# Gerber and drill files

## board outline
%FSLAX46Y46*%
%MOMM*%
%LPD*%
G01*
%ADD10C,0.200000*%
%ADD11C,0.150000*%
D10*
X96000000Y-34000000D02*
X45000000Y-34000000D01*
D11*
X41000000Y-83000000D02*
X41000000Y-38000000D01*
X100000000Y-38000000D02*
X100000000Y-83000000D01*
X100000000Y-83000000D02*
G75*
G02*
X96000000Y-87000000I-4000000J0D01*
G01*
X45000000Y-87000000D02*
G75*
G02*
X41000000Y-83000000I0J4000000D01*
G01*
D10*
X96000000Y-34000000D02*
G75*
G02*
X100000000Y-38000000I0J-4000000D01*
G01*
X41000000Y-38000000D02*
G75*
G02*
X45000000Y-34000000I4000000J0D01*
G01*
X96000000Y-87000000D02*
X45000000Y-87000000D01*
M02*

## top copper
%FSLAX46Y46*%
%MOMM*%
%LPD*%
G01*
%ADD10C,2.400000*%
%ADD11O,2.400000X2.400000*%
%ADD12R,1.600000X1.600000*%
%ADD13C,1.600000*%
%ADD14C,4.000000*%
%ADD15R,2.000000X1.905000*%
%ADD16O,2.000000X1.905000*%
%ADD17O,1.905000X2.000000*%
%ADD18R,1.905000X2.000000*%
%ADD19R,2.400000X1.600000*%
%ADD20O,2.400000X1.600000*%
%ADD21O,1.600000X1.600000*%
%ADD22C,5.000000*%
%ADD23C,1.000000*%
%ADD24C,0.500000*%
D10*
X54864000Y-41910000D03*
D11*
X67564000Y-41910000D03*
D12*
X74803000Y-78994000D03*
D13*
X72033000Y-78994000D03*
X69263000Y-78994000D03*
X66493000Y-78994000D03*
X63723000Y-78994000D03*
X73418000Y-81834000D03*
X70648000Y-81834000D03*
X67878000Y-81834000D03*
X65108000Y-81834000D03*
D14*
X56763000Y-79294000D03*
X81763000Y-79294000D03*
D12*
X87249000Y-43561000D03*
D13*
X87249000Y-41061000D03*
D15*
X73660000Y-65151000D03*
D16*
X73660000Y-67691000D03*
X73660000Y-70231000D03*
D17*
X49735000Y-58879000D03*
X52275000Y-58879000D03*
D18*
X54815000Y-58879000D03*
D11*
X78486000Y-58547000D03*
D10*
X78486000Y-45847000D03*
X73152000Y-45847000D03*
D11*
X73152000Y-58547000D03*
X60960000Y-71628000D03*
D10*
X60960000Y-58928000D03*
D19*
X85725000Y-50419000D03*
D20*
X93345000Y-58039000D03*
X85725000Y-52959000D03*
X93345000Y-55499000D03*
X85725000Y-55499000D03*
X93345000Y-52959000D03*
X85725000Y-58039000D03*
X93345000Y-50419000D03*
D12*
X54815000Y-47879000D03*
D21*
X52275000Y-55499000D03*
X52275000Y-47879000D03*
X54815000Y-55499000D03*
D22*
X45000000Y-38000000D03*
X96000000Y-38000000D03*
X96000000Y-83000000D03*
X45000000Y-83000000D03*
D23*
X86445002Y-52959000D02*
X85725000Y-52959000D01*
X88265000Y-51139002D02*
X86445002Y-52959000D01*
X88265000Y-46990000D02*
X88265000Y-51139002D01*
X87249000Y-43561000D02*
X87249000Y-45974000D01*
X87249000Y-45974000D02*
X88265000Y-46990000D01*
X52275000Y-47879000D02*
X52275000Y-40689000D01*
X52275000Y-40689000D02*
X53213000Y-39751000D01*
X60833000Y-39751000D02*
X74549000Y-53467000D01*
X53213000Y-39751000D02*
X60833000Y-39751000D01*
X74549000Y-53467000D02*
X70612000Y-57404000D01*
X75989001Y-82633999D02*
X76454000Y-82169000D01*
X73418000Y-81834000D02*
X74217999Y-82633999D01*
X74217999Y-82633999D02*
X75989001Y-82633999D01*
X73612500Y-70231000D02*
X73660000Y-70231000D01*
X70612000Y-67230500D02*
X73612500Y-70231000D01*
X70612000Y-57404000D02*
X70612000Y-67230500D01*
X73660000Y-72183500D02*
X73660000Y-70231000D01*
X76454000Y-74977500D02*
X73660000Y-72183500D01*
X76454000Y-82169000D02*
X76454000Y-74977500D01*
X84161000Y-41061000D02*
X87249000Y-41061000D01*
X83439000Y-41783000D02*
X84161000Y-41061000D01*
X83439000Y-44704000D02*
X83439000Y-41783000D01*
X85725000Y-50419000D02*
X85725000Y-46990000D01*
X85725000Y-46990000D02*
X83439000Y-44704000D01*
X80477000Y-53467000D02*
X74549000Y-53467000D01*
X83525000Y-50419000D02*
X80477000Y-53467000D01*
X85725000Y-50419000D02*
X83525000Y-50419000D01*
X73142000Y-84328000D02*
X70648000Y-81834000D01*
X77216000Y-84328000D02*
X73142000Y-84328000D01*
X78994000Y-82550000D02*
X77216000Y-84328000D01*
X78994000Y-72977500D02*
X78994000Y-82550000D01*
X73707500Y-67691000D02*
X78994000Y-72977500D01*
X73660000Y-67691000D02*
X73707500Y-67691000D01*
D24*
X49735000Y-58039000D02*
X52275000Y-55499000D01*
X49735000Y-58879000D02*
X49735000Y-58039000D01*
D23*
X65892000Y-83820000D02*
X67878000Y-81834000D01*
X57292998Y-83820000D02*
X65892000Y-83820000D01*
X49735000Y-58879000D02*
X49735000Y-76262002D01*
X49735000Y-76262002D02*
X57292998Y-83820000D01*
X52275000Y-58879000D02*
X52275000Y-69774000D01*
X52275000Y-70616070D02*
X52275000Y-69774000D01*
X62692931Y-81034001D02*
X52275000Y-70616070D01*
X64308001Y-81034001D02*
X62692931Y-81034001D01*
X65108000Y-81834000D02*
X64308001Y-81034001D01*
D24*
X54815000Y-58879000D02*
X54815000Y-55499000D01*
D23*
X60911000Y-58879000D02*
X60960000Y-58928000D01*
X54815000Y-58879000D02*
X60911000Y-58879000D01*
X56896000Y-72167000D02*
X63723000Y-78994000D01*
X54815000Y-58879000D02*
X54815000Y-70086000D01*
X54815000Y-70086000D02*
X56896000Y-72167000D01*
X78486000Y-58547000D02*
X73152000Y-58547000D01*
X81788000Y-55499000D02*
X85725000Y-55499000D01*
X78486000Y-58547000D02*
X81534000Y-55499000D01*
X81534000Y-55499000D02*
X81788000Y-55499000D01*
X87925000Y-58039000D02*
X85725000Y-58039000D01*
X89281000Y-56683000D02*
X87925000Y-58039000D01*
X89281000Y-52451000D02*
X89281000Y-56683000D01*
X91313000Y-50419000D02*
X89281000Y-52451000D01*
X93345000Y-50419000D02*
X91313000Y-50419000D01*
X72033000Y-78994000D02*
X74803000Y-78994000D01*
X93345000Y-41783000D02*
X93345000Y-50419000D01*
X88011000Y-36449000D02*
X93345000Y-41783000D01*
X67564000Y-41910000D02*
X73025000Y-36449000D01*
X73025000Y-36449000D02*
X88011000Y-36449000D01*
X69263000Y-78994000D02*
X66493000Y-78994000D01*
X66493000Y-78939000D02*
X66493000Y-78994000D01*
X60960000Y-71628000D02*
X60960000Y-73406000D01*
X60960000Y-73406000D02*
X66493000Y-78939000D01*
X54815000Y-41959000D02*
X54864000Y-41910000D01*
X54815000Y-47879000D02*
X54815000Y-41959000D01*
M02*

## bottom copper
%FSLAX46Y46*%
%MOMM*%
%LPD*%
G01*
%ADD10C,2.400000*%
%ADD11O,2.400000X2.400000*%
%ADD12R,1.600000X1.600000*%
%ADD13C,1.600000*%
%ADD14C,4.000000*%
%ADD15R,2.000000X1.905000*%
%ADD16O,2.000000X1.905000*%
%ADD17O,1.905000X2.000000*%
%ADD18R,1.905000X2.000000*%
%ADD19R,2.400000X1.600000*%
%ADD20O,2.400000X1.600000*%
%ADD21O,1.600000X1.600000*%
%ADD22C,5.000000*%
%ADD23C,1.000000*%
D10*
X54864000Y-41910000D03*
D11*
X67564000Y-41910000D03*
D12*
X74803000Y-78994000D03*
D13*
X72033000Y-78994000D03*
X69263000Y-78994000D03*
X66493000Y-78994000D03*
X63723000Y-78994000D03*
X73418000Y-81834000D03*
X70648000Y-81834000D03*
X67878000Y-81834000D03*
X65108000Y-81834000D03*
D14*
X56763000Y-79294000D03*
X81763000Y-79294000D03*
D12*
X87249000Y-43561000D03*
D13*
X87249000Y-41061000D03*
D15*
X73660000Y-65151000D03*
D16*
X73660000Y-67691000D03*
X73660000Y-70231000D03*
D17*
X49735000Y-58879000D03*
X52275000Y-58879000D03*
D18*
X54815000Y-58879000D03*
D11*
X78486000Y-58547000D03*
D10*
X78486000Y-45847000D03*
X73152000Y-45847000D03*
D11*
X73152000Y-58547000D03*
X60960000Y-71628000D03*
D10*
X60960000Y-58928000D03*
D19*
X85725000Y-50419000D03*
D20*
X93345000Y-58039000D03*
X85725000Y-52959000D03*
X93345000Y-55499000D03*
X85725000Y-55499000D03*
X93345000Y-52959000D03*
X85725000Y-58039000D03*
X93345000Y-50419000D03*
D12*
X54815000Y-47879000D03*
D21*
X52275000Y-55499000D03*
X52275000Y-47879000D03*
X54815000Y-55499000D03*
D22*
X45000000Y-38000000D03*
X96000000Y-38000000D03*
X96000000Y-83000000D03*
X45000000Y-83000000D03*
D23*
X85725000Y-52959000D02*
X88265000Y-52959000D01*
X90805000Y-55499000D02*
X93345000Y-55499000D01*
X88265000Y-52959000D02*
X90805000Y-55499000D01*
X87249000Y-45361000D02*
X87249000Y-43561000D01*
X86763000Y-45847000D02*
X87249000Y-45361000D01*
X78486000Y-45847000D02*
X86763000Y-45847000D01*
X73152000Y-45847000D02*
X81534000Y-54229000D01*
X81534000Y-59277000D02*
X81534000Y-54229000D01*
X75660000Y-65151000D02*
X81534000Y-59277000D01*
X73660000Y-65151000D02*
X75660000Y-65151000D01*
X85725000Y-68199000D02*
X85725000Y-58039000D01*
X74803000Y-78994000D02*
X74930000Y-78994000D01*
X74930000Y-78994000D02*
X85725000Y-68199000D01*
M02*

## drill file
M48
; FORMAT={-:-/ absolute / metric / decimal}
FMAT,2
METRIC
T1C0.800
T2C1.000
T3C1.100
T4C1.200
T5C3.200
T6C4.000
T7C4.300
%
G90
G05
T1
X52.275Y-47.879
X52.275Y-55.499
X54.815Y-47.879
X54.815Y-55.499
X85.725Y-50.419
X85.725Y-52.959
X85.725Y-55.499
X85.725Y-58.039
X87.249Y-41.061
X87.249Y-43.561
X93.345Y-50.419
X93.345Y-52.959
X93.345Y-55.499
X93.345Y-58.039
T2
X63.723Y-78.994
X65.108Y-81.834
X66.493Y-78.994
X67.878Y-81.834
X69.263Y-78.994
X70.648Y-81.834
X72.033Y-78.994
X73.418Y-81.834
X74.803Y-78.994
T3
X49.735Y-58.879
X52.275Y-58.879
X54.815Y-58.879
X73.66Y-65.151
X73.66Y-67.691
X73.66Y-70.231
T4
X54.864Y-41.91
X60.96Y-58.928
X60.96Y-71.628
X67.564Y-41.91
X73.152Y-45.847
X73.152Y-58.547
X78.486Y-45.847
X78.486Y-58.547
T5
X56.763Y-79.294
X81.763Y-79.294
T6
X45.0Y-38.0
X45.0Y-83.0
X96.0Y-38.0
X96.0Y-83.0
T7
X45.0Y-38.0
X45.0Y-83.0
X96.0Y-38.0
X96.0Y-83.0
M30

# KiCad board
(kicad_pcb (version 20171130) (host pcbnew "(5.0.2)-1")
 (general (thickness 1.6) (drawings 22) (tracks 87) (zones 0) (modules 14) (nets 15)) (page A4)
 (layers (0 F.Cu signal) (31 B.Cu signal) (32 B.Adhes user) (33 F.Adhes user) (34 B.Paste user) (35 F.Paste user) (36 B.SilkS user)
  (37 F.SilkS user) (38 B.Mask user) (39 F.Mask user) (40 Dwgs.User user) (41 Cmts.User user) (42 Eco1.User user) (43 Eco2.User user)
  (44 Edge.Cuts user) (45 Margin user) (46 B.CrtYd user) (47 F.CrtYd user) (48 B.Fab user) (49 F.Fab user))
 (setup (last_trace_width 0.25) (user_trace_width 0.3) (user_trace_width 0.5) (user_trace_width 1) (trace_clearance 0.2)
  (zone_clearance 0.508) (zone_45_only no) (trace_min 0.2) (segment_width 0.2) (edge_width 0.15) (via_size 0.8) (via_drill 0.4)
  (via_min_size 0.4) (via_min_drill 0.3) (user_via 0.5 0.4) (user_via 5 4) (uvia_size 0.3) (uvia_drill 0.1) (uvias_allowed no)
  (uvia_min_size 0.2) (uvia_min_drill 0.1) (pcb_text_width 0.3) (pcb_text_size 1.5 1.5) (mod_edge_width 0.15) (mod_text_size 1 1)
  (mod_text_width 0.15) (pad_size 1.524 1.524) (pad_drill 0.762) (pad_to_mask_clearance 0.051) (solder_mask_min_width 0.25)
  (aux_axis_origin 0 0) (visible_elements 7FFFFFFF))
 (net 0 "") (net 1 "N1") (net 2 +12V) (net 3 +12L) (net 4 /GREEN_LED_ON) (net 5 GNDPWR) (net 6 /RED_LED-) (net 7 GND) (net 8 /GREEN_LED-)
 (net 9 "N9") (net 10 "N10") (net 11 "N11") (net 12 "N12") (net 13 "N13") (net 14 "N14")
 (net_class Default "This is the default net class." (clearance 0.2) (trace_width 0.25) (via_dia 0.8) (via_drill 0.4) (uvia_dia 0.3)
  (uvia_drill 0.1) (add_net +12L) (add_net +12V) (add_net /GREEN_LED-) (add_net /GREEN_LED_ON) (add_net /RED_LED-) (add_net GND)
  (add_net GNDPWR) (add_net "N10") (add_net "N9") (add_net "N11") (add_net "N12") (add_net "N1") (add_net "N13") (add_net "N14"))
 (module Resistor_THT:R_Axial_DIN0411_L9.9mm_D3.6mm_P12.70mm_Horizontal (layer F.Cu) (at 54.864 41.91)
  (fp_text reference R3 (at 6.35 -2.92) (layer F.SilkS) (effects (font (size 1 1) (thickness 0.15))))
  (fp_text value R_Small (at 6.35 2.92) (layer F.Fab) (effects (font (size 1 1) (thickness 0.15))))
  (pad 1 thru_hole circle (at 0 0) (size 2.4 2.4) (drill 1.2) (layers *.Cu *.Mask) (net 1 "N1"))
  (pad 2 thru_hole oval (at 12.7 0) (size 2.4 2.4) (drill 1.2) (layers *.Cu *.Mask) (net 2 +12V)))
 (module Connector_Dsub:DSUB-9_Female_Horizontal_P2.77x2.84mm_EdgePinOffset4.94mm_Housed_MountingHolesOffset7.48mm (layer F.Cu)
  (at 74.803 78.994)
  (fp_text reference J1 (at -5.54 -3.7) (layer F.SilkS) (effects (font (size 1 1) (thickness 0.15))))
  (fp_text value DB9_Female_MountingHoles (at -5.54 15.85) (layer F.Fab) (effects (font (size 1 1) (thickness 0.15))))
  (pad 1 thru_hole rect (at 0 0) (size 1.6 1.6) (drill 1) (layers *.Cu *.Mask) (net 2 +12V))
  (pad 2 thru_hole circle (at -2.77 0) (size 1.6 1.6) (drill 1) (layers *.Cu *.Mask) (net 2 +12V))
  (pad 3 thru_hole circle (at -5.54 0) (size 1.6 1.6) (drill 1) (layers *.Cu *.Mask) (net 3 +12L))
  (pad 4 thru_hole circle (at -8.31 0) (size 1.6 1.6) (drill 1) (layers *.Cu *.Mask) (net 3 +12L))
  (pad 5 thru_hole circle (at -11.08 0) (size 1.6 1.6) (drill 1) (layers *.Cu *.Mask) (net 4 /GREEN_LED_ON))
  (pad 6 thru_hole circle (at -1.385 2.84) (size 1.6 1.6) (drill 1) (layers *.Cu *.Mask) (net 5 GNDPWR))
  (pad 7 thru_hole circle (at -4.155 2.84) (size 1.6 1.6) (drill 1) (layers *.Cu *.Mask) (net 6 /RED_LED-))
  (pad 8 thru_hole circle (at -6.925 2.84) (size 1.6 1.6) (drill 1) (layers *.Cu *.Mask) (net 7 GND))
  (pad 9 thru_hole circle (at -9.695 2.84) (size 1.6 1.6) (drill 1) (layers *.Cu *.Mask) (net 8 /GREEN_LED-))
  (pad 0 thru_hole circle (at -18.04 0.3) (size 4 4) (drill 3.2) (layers *.Cu *.Mask) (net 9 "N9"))
  (pad 0 thru_hole circle (at 6.96 0.3) (size 4 4) (drill 3.2) (layers *.Cu *.Mask) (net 9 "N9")))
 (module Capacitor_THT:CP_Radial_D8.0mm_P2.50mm (layer F.Cu) (at 87.249 43.561 90)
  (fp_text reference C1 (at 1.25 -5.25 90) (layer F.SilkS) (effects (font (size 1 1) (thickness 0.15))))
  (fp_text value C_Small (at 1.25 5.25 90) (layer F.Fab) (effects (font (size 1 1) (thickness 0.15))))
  (pad 1 thru_hole rect (at 0 0 90) (size 1.6 1.6) (drill 0.8) (layers *.Cu *.Mask) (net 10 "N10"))
  (pad 2 thru_hole circle (at 2.5 0 90) (size 1.6 1.6) (drill 0.8) (layers *.Cu *.Mask) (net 5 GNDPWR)))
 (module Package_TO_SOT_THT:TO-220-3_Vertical (layer F.Cu) (at 73.66 65.151 270)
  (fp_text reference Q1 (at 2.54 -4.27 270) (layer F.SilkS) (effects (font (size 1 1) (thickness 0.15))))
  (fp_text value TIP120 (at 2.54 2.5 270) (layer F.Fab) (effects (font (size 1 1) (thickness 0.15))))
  (pad 1 thru_hole rect (at 0 0 270) (size 1.905 2) (drill 1.1) (layers *.Cu *.Mask) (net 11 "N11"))
  (pad 2 thru_hole oval (at 2.54 0 270) (size 1.905 2) (drill 1.1) (layers *.Cu *.Mask) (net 6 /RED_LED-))
  (pad 3 thru_hole oval (at 5.08 0 270) (size 1.905 2) (drill 1.1) (layers *.Cu *.Mask) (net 5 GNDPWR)))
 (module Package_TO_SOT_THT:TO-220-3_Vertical (layer F.Cu) (at 54.815 58.879 180)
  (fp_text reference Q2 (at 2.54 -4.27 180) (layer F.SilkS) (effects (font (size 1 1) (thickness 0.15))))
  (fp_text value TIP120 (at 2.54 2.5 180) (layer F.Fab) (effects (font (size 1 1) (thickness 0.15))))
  (pad 3 thru_hole oval (at 5.08 0 180) (size 1.905 2) (drill 1.1) (layers *.Cu *.Mask) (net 7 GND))
  (pad 2 thru_hole oval (at 2.54 0 180) (size 1.905 2) (drill 1.1) (layers *.Cu *.Mask) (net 8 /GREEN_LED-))
  (pad 1 thru_hole rect (at 0 0 180) (size 1.905 2) (drill 1.1) (layers *.Cu *.Mask) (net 4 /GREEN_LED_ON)))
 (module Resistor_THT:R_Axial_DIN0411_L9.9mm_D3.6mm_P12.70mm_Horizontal (layer F.Cu) (at 78.486 45.847 270)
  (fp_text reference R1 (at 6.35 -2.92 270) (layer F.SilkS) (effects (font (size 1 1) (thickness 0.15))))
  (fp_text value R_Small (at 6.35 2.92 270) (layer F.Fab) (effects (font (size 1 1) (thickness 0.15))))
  (pad 2 thru_hole oval (at 12.7 0 270) (size 2.4 2.4) (drill 1.2) (layers *.Cu *.Mask) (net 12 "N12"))
  (pad 1 thru_hole circle (at 0 0 270) (size 2.4 2.4) (drill 1.2) (layers *.Cu *.Mask) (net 10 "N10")))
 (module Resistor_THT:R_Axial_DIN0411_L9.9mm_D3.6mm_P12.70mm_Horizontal (layer F.Cu) (at 73.152 45.847 270)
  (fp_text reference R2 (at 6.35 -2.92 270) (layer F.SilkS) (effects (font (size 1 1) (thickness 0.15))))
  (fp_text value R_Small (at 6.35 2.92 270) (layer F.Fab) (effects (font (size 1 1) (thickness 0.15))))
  (pad 1 thru_hole circle (at 0 0 270) (size 2.4 2.4) (drill 1.2) (layers *.Cu *.Mask) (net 11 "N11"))
  (pad 2 thru_hole oval (at 12.7 0 270) (size 2.4 2.4) (drill 1.2) (layers *.Cu *.Mask) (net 12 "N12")))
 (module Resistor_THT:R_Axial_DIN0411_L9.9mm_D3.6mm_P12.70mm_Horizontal (layer F.Cu) (at 60.96 58.928 270)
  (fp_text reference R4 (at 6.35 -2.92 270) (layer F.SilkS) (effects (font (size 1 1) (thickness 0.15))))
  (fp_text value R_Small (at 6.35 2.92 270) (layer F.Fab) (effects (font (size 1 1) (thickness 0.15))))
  (pad 2 thru_hole oval (at 12.7 0 270) (size 2.4 2.4) (drill 1.2) (layers *.Cu *.Mask) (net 3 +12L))
  (pad 1 thru_hole circle (at 0 0 270) (size 2.4 2.4) (drill 1.2) (layers *.Cu *.Mask) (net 4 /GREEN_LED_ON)))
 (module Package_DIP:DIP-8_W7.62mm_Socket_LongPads (layer F.Cu) (at 85.725 50.419)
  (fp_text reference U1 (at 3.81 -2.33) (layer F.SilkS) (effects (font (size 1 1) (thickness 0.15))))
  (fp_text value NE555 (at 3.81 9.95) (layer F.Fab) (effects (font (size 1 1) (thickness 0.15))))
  (pad 1 thru_hole rect (at 0 0) (size 2.4 1.6) (drill 0.8) (layers *.Cu *.Mask) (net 5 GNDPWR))
  (pad 5 thru_hole oval (at 7.62 7.62) (size 2.4 1.6) (drill 0.8) (layers *.Cu *.Mask) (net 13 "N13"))
  (pad 2 thru_hole oval (at 0 2.54) (size 2.4 1.6) (drill 0.8) (layers *.Cu *.Mask) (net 10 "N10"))
  (pad 6 thru_hole oval (at 7.62 5.08) (size 2.4 1.6) (drill 0.8) (layers *.Cu *.Mask) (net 10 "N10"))
  (pad 3 thru_hole oval (at 0 5.08) (size 2.4 1.6) (drill 0.8) (layers *.Cu *.Mask) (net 12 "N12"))
  (pad 7 thru_hole oval (at 7.62 2.54) (size 2.4 1.6) (drill 0.8) (layers *.Cu *.Mask) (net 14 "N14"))
  (pad 4 thru_hole oval (at 0 7.62) (size 2.4 1.6) (drill 0.8) (layers *.Cu *.Mask) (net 2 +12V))
  (pad 8 thru_hole oval (at 7.62 0) (size 2.4 1.6) (drill 0.8) (layers *.Cu *.Mask) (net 2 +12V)))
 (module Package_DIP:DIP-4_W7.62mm (layer F.Cu) (at 54.815 47.879 270)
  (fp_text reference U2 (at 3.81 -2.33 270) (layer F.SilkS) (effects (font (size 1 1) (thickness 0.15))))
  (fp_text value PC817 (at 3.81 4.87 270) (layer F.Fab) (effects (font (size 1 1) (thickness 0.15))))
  (pad 1 thru_hole rect (at 0 0 270) (size 1.6 1.6) (drill 0.8) (layers *.Cu *.Mask) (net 1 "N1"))
  (pad 3 thru_hole oval (at 7.62 2.54 270) (size 1.6 1.6) (drill 0.8) (layers *.Cu *.Mask) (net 7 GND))
  (pad 2 thru_hole oval (at 0 2.54 270) (size 1.6 1.6) (drill 0.8) (layers *.Cu *.Mask) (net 5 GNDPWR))
  (pad 4 thru_hole oval (at 7.62 0 270) (size 1.6 1.6) (drill 0.8) (layers *.Cu *.Mask) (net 4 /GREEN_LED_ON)))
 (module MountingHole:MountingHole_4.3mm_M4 (layer F.Cu) (at 96 38)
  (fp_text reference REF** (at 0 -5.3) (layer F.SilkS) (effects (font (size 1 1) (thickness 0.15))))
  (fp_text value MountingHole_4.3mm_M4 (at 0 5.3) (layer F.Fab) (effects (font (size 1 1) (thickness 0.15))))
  (pad 1 np_thru_hole circle (at 0 0) (size 4.3 4.3) (drill 4.3) (layers *.Cu *.Mask)))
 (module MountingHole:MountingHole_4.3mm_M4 (layer F.Cu) (at 45 38)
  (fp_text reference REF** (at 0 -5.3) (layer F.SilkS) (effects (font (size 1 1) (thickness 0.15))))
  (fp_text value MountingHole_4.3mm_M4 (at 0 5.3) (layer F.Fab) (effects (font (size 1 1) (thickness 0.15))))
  (pad 1 np_thru_hole circle (at 0 0) (size 4.3 4.3) (drill 4.3) (layers *.Cu *.Mask)))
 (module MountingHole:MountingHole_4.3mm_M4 (layer F.Cu) (at 45 83)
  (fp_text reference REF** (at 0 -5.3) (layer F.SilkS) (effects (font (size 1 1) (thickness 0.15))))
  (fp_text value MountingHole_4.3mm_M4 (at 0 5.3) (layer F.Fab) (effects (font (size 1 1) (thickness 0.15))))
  (pad 1 np_thru_hole circle (at 0 0) (size 4.3 4.3) (drill 4.3) (layers *.Cu *.Mask)))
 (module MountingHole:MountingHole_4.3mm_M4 (layer F.Cu) (at 96 83)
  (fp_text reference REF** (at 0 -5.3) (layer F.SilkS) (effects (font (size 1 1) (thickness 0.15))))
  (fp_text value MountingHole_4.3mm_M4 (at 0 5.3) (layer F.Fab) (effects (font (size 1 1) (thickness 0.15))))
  (pad 1 np_thru_hole circle (at 0 0) (size 4.3 4.3) (drill 4.3) (layers *.Cu *.Mask)))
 (gr_line (start 96 34) (end 45 34) (layer Edge.Cuts) (width 0.2))
 (gr_line (start 41 83) (end 41 38) (layer Edge.Cuts) (width 0.15))
 (gr_line (start 100 38) (end 100 83) (layer Edge.Cuts) (width 0.15))
 (gr_arc (start 96 83) (end 96 87) (angle -90) (layer Edge.Cuts) (width 0.15))
 (gr_arc (start 45 83) (end 41 83) (angle -90) (layer Edge.Cuts) (width 0.15))
 (gr_arc (start 96 38) (end 100 38) (angle -90) (layer Edge.Cuts) (width 0.2))
 (gr_arc (start 45 38) (end 45 34) (angle -90) (layer Edge.Cuts) (width 0.2))
 (gr_line (start 96 87) (end 45 87) (layer Edge.Cuts) (width 0.2))
 (via (at 45 38) (size 5) (drill 4) (layers F.Cu B.Cu) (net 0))
 (via (at 96 38) (size 5) (drill 4) (layers F.Cu B.Cu) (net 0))
 (via (at 96 83) (size 5) (drill 4) (layers F.Cu B.Cu) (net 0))
 (via (at 45 83) (size 5) (drill 4) (layers F.Cu B.Cu) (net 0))
 (segment (start 85.725 52.959) (end 88.265 52.959) (width 1) (layer B.Cu) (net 10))
 (segment (start 90.805 55.499) (end 93.345 55.499) (width 1) (layer B.Cu) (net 10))
 (segment (start 88.265 52.959) (end 90.805 55.499) (width 1) (layer B.Cu) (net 10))
 (segment (start 87.249 45.361) (end 87.249 43.561) (width 1) (layer B.Cu) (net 10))
 (segment (start 86.763 45.847) (end 87.249 45.361) (width 1) (layer B.Cu) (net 10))
 (segment (start 78.486 45.847) (end 86.763 45.847) (width 1) (layer B.Cu) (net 10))
 (segment (start 86.445002 52.959) (end 85.725 52.959) (width 1) (layer F.Cu) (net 10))
 (segment (start 88.265 51.139002) (end 86.445002 52.959) (width 1) (layer F.Cu) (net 10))
 (segment (start 88.265 46.99) (end 88.265 51.139002) (width 1) (layer F.Cu) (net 10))
 (segment (start 87.249 43.561) (end 87.249 45.974) (width 1) (layer F.Cu) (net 10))
 (segment (start 87.249 45.974) (end 88.265 46.99) (width 1) (layer F.Cu) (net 10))
 (segment (start 52.275 47.879) (end 52.275 40.689) (width 1) (layer F.Cu) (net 5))
 (segment (start 52.275 40.689) (end 53.213 39.751) (width 1) (layer F.Cu) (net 5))
 (segment (start 60.833 39.751) (end 74.549 53.467) (width 1) (layer F.Cu) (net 5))
 (segment (start 53.213 39.751) (end 60.833 39.751) (width 1) (layer F.Cu) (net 5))
 (segment (start 74.549 53.467) (end 70.612 57.404) (width 1) (layer F.Cu) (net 5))
 (segment (start 75.989001 82.633999) (end 76.454 82.169) (width 1) (layer F.Cu) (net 5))
 (segment (start 73.418 81.834) (end 74.217999 82.633999) (width 1) (layer F.Cu) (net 5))
 (segment (start 74.217999 82.633999) (end 75.989001 82.633999) (width 1) (layer F.Cu) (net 5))
 (segment (start 73.6125 70.231) (end 73.66 70.231) (width 1) (layer F.Cu) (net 5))
 (segment (start 70.612 67.2305) (end 73.6125 70.231) (width 1) (layer F.Cu) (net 5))
 (segment (start 70.612 57.404) (end 70.612 67.2305) (width 1) (layer F.Cu) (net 5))
 (segment (start 73.66 72.1835) (end 73.66 70.231) (width 1) (layer F.Cu) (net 5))
 (segment (start 76.454 74.9775) (end 73.66 72.1835) (width 1) (layer F.Cu) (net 5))
 (segment (start 76.454 82.169) (end 76.454 74.9775) (width 1) (layer F.Cu) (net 5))
 (segment (start 84.161 41.061) (end 87.249 41.061) (width 1) (layer F.Cu) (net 5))
 (segment (start 83.439 41.783) (end 84.161 41.061) (width 1) (layer F.Cu) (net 5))
 (segment (start 83.439 44.704) (end 83.439 41.783) (width 1) (layer F.Cu) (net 5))
 (segment (start 85.725 50.419) (end 85.725 46.99) (width 1) (layer F.Cu) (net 5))
 (segment (start 85.725 46.99) (end 83.439 44.704) (width 1) (layer F.Cu) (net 5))
 (segment (start 80.477 53.467) (end 74.549 53.467) (width 1) (layer F.Cu) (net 5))
 (segment (start 83.525 50.419) (end 80.477 53.467) (width 1) (layer F.Cu) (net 5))
 (segment (start 85.725 50.419) (end 83.525 50.419) (width 1) (layer F.Cu) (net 5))
 (segment (start 73.152 45.847) (end 81.534 54.229) (width 1) (layer B.Cu) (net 11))
 (segment (start 81.534 59.277) (end 81.534 54.229) (width 1) (layer B.Cu) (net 11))
 (segment (start 75.66 65.151) (end 81.534 59.277) (width 1) (layer B.Cu) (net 11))
 (segment (start 73.66 65.151) (end 75.66 65.151) (width 1) (layer B.Cu) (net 11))
 (segment (start 73.142 84.328) (end 70.648 81.834) (width 1) (layer F.Cu) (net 6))
 (segment (start 77.216 84.328) (end 73.142 84.328) (width 1) (layer F.Cu) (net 6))
 (segment (start 78.994 82.55) (end 77.216 84.328) (width 1) (layer F.Cu) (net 6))
 (segment (start 78.994 72.9775) (end 78.994 82.55) (width 1) (layer F.Cu) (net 6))
 (segment (start 73.7075 67.691) (end 78.994 72.9775) (width 1) (layer F.Cu) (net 6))
 (segment (start 73.66 67.691) (end 73.7075 67.691) (width 1) (layer F.Cu) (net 6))
 (segment (start 49.735 58.039) (end 52.275 55.499) (width 0.5) (layer F.Cu) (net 7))
 (segment (start 49.735 58.879) (end 49.735 58.039) (width 0.5) (layer F.Cu) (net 7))
 (segment (start 65.892 83.82) (end 67.878 81.834) (width 1) (layer F.Cu) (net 7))
 (segment (start 57.292998 83.82) (end 65.892 83.82) (width 1) (layer F.Cu) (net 7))
 (segment (start 49.735 58.879) (end 49.735 76.262002) (width 1) (layer F.Cu) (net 7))
 (segment (start 49.735 76.262002) (end 57.292998 83.82) (width 1) (layer F.Cu) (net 7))
 (segment (start 52.275 58.879) (end 52.275 69.774) (width 1) (layer F.Cu) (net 8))
 (segment (start 52.275 70.61607) (end 52.275 69.774) (width 1) (layer F.Cu) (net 8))
 (segment (start 62.692931 81.034001) (end 52.275 70.61607) (width 1) (layer F.Cu) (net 8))
 (segment (start 64.308001 81.034001) (end 62.692931 81.034001) (width 1) (layer F.Cu) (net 8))
 (segment (start 65.108 81.834) (end 64.308001 81.034001) (width 1) (layer F.Cu) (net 8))
 (segment (start 54.815 58.879) (end 54.815 55.499) (width 0.5) (layer F.Cu) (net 4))
 (segment (start 60.911 58.879) (end 60.96 58.928) (width 1) (layer F.Cu) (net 4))
 (segment (start 54.815 58.879) (end 60.911 58.879) (width 1) (layer F.Cu) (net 4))
 (segment (start 56.896 72.167) (end 63.723 78.994) (width 1) (layer F.Cu) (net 4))
 (segment (start 54.815 58.879) (end 54.815 70.086) (width 1) (layer F.Cu) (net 4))
 (segment (start 54.815 70.086) (end 56.896 72.167) (width 1) (layer F.Cu) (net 4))
 (segment (start 78.486 58.547) (end 73.152 58.547) (width 1) (layer F.Cu) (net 12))
 (segment (start 81.788 55.499) (end 85.725 55.499) (width 1) (layer F.Cu) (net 12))
 (segment (start 78.486 58.547) (end 81.534 55.499) (width 1) (layer F.Cu) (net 12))
 (segment (start 81.534 55.499) (end 81.788 55.499) (width 1) (layer F.Cu) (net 12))
 (segment (start 87.925 58.039) (end 85.725 58.039) (width 1) (layer F.Cu) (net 2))
 (segment (start 89.281 56.683) (end 87.925 58.039) (width 1) (layer F.Cu) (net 2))
 (segment (start 89.281 52.451) (end 89.281 56.683) (width 1) (layer F.Cu) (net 2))
 (segment (start 91.313 50.419) (end 89.281 52.451) (width 1) (layer F.Cu) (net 2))
 (segment (start 93.345 50.419) (end 91.313 50.419) (width 1) (layer F.Cu) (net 2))
 (segment (start 72.033 78.994) (end 74.803 78.994) (width 1) (layer F.Cu) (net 2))
 (segment (start 93.345 41.783) (end 93.345 50.419) (width 1) (layer F.Cu) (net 2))
 (segment (start 88.011 36.449) (end 93.345 41.783) (width 1) (layer F.Cu) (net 2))
 (segment (start 67.564 41.91) (end 73.025 36.449) (width 1) (layer F.Cu) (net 2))
 (segment (start 73.025 36.449) (end 88.011 36.449) (width 1) (layer F.Cu) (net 2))
 (segment (start 85.725 68.199) (end 85.725 58.039) (width 1) (layer B.Cu) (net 2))
 (segment (start 74.803 78.994) (end 74.93 78.994) (width 1) (layer B.Cu) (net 2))
 (segment (start 74.93 78.994) (end 85.725 68.199) (width 1) (layer B.Cu) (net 2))
 (segment (start 69.263 78.994) (end 66.493 78.994) (width 1) (layer F.Cu) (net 3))
 (segment (start 66.493 78.939) (end 66.493 78.994) (width 1) (layer F.Cu) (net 3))
 (segment (start 60.96 71.628) (end 60.96 73.406) (width 1) (layer F.Cu) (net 3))
 (segment (start 60.96 73.406) (end 66.493 78.939) (width 1) (layer F.Cu) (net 3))
 (segment (start 54.815 41.959) (end 54.864 41.91) (width 1) (layer F.Cu) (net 1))
 (segment (start 54.815 47.879) (end 54.815 41.959) (width 1) (layer F.Cu) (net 1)))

